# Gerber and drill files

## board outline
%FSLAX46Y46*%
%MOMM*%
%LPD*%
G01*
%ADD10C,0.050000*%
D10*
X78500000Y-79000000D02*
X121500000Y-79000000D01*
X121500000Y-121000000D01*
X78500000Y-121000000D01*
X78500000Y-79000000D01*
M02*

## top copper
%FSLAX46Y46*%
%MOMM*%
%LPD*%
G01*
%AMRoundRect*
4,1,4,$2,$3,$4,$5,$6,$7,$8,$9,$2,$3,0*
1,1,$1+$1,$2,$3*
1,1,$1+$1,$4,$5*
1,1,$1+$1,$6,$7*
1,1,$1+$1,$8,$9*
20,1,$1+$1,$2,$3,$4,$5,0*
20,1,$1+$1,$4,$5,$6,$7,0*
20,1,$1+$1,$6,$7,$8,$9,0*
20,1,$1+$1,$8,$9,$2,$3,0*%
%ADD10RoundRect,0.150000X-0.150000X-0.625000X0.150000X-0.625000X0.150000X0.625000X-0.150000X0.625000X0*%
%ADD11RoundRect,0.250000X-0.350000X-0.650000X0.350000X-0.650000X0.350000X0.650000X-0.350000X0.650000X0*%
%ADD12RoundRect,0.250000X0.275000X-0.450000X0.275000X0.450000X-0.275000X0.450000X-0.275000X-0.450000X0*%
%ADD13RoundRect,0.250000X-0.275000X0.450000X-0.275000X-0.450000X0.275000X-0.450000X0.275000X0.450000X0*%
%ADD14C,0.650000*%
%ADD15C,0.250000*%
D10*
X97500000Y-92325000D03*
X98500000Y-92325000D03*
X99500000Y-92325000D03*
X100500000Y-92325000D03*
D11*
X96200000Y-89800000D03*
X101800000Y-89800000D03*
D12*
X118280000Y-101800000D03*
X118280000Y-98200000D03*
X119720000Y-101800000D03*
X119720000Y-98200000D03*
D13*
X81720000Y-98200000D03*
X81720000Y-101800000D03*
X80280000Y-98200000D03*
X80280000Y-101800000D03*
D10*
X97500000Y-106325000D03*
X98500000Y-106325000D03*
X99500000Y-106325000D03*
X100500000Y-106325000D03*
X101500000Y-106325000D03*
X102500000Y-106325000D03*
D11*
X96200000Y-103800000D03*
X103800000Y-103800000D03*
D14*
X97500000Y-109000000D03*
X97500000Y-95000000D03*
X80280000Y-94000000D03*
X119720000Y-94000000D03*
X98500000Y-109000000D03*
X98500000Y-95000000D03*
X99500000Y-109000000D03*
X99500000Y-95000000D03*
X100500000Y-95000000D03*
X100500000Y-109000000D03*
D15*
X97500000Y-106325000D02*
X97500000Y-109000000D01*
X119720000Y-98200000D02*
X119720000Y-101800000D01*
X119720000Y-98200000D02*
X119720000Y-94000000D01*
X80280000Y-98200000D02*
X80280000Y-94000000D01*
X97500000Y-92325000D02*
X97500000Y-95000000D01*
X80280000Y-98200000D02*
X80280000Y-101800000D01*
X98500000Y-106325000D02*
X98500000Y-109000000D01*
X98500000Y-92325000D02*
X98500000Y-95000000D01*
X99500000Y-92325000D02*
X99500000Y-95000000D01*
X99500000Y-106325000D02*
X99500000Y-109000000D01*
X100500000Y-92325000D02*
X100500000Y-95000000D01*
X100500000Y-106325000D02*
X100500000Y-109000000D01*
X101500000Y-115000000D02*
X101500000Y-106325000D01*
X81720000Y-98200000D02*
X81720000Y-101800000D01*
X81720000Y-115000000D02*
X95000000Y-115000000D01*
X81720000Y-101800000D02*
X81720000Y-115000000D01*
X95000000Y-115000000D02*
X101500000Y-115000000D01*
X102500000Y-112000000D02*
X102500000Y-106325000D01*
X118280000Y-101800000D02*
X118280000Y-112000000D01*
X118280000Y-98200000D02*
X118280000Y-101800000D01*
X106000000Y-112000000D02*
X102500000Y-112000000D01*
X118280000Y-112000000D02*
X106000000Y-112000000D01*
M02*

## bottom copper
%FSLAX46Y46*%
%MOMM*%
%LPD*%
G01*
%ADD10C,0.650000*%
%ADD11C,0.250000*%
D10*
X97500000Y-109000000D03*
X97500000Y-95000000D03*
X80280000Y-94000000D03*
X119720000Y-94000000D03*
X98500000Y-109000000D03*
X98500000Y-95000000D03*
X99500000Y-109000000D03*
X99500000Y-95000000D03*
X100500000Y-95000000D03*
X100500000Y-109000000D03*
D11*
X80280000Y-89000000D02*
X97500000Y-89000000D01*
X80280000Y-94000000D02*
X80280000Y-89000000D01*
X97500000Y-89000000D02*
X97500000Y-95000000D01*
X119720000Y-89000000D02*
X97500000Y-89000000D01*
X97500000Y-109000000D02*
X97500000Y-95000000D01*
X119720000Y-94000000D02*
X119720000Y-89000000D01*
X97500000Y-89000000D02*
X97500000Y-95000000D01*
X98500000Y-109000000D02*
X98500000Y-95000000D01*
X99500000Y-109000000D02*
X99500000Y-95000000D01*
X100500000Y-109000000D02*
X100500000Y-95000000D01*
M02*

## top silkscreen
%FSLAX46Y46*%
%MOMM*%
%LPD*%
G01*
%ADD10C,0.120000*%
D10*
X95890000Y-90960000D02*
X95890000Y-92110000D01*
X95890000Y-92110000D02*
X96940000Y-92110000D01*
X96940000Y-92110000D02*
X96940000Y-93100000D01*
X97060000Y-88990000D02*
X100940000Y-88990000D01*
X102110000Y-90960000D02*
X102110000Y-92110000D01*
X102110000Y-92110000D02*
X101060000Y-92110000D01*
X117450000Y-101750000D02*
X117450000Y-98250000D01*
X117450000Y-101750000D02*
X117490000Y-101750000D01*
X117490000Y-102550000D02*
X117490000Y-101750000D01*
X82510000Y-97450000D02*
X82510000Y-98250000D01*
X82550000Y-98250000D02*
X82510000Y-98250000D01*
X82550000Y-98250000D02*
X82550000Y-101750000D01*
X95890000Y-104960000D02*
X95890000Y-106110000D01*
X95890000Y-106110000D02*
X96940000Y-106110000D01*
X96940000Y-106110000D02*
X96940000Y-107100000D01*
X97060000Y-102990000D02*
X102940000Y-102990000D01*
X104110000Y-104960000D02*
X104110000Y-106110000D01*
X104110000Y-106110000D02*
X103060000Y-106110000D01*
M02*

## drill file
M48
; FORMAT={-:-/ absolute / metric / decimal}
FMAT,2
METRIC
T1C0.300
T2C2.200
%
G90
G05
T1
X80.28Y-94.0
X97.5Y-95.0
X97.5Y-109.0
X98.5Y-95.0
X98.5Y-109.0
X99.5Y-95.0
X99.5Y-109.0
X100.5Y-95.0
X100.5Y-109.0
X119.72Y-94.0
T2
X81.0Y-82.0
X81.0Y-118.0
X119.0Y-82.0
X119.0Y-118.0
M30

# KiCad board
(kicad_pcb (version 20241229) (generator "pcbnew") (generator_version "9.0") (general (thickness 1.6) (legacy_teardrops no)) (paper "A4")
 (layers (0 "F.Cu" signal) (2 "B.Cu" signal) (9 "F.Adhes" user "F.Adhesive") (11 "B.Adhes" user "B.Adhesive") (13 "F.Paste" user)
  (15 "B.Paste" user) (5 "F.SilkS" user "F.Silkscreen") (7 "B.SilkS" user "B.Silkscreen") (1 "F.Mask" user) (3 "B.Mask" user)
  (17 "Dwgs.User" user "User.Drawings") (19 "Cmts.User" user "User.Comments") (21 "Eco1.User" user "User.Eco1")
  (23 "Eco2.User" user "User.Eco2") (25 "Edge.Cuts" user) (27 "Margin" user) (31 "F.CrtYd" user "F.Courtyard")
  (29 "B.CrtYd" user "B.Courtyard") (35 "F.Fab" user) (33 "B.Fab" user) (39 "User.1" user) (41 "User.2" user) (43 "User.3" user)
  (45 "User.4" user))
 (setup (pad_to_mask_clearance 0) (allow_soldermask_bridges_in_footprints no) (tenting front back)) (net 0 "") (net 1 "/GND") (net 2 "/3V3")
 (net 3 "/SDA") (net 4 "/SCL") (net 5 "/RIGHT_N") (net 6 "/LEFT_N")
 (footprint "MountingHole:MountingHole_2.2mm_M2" (layer "F.Cu") (at 119 82)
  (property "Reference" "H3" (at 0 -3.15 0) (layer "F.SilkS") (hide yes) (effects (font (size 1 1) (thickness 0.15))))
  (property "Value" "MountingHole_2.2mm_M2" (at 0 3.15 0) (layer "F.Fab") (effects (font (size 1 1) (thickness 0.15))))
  (pad "" np_thru_hole circle (at 0 0) (size 2.2 2.2) (drill 2.2) (layers "*.Cu" "*.Mask")))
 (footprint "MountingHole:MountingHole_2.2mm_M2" (layer "F.Cu") (at 81 82)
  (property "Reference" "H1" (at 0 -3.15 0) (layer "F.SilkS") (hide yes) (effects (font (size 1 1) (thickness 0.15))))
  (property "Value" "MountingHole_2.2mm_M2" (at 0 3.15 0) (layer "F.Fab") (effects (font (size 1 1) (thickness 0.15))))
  (pad "" np_thru_hole circle (at 0 0) (size 2.2 2.2) (drill 2.2) (layers "*.Cu" "*.Mask")))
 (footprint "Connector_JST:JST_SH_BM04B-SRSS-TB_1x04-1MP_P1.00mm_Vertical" (layer "F.Cu") (at 99 91)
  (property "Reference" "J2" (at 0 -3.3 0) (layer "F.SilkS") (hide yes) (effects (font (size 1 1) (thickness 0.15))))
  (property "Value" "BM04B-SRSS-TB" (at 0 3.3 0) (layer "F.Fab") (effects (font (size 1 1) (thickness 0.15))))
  (fp_line (start -3.11 -0.04) (end -3.11 1.11) (stroke (width 0.12) (type solid)) (layer "F.SilkS"))
  (fp_line (start -3.11 1.11) (end -2.06 1.11) (stroke (width 0.12) (type solid)) (layer "F.SilkS"))
  (fp_line (start -2.06 1.11) (end -2.06 2.1) (stroke (width 0.12) (type solid)) (layer "F.SilkS"))
  (fp_line (start -1.94 -2.01) (end 1.94 -2.01) (stroke (width 0.12) (type solid)) (layer "F.SilkS"))
  (fp_line (start 3.11 -0.04) (end 3.11 1.11) (stroke (width 0.12) (type solid)) (layer "F.SilkS"))
  (fp_line (start 3.11 1.11) (end 2.06 1.11) (stroke (width 0.12) (type solid)) (layer "F.SilkS"))
  (pad "1" smd roundrect (at -1.5 1.325) (size 0.6 1.55) (layers "F.Cu" "F.Mask" "F.Paste") (roundrect_rratio 0.25) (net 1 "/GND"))
  (pad "2" smd roundrect (at -0.5 1.325) (size 0.6 1.55) (layers "F.Cu" "F.Mask" "F.Paste") (roundrect_rratio 0.25) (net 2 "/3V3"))
  (pad "3" smd roundrect (at 0.5 1.325) (size 0.6 1.55) (layers "F.Cu" "F.Mask" "F.Paste") (roundrect_rratio 0.25) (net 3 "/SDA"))
  (pad "4" smd roundrect (at 1.5 1.325) (size 0.6 1.55) (layers "F.Cu" "F.Mask" "F.Paste") (roundrect_rratio 0.25) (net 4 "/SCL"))
  (pad "MP" smd roundrect (at -2.8 -1.2) (size 1.2 1.8) (layers "F.Cu" "F.Mask" "F.Paste") (roundrect_rratio 0.208333))
  (pad "MP" smd roundrect (at 2.8 -1.2) (size 1.2 1.8) (layers "F.Cu" "F.Mask" "F.Paste") (roundrect_rratio 0.208333)))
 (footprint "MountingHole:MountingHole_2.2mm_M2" (layer "F.Cu") (at 81 118)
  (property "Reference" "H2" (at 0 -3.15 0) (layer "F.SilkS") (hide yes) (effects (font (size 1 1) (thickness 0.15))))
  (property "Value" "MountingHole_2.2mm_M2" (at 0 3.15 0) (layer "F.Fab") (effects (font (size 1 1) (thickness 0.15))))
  (pad "" np_thru_hole circle (at 0 0) (size 2.2 2.2) (drill 2.2) (layers "*.Cu" "*.Mask")))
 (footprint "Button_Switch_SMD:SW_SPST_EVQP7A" (layer "F.Cu") (at 119 100 90)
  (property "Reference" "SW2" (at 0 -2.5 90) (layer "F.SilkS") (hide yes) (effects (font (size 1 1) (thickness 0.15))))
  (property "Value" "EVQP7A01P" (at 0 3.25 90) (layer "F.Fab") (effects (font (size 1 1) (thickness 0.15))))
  (fp_line (start -1.75 -1.55) (end 1.75 -1.55) (stroke (width 0.12) (type solid)) (layer "F.SilkS"))
  (fp_line (start -1.75 -1.55) (end -1.75 -1.51) (stroke (width 0.12) (type default)) (layer "F.SilkS"))
  (fp_line (start -2.55 -1.51) (end -1.75 -1.51) (stroke (width 0.12) (type default)) (layer "F.SilkS"))
  (pad "1" smd roundrect (at -1.8 -0.72 90) (size 1.4 1.05) (layers "F.Cu" "F.Mask" "F.Paste") (roundrect_rratio 0.2380952381)
   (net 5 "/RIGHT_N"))
  (pad "1" smd roundrect (at 1.8 -0.72 90) (size 1.4 1.05) (layers "F.Cu" "F.Mask" "F.Paste") (roundrect_rratio 0.2380952381)
   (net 5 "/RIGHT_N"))
  (pad "2" smd roundrect (at -1.8 0.72 90) (size 1.4 1.05) (layers "F.Cu" "F.Mask" "F.Paste") (roundrect_rratio 0.2380952381) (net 1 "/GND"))
  (pad "2" smd roundrect (at 1.8 0.72 90) (size 1.4 1.05) (layers "F.Cu" "F.Mask" "F.Paste") (roundrect_rratio 0.2380952381) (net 1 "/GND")))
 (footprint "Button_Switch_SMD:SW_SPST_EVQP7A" (layer "F.Cu") (at 81 100 -90)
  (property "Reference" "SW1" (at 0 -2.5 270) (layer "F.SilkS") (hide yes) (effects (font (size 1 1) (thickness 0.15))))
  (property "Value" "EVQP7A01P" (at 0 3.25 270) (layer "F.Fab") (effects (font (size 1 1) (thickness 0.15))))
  (fp_line (start -2.55 -1.51) (end -1.75 -1.51) (stroke (width 0.12) (type default)) (layer "F.SilkS"))
  (fp_line (start -1.75 -1.55) (end -1.75 -1.51) (stroke (width 0.12) (type default)) (layer "F.SilkS"))
  (fp_line (start -1.75 -1.55) (end 1.75 -1.55) (stroke (width 0.12) (type solid)) (layer "F.SilkS"))
  (pad "1" smd roundrect (at -1.8 -0.72 270) (size 1.4 1.05) (layers "F.Cu" "F.Mask" "F.Paste") (roundrect_rratio 0.2380952381)
   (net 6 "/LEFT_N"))
  (pad "1" smd roundrect (at 1.8 -0.72 270) (size 1.4 1.05) (layers "F.Cu" "F.Mask" "F.Paste") (roundrect_rratio 0.2380952381)
   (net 6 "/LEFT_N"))
  (pad "2" smd roundrect (at -1.8 0.72 270) (size 1.4 1.05) (layers "F.Cu" "F.Mask" "F.Paste") (roundrect_rratio 0.2380952381)
   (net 1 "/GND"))
  (pad "2" smd roundrect (at 1.8 0.72 270) (size 1.4 1.05) (layers "F.Cu" "F.Mask" "F.Paste") (roundrect_rratio 0.2380952381) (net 1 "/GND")))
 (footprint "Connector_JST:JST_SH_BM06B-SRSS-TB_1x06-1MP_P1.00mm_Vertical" (layer "F.Cu") (at 100 105)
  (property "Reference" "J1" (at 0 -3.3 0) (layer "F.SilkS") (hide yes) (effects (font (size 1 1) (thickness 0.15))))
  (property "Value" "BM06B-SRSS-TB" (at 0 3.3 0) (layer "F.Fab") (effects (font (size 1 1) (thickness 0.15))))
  (fp_line (start -4.11 -0.04) (end -4.11 1.11) (stroke (width 0.12) (type solid)) (layer "F.SilkS"))
  (fp_line (start -4.11 1.11) (end -3.06 1.11) (stroke (width 0.12) (type solid)) (layer "F.SilkS"))
  (fp_line (start -3.06 1.11) (end -3.06 2.1) (stroke (width 0.12) (type solid)) (layer "F.SilkS"))
  (fp_line (start -2.94 -2.01) (end 2.94 -2.01) (stroke (width 0.12) (type solid)) (layer "F.SilkS"))
  (fp_line (start 4.11 -0.04) (end 4.11 1.11) (stroke (width 0.12) (type solid)) (layer "F.SilkS"))
  (fp_line (start 4.11 1.11) (end 3.06 1.11) (stroke (width 0.12) (type solid)) (layer "F.SilkS"))
  (pad "1" smd roundrect (at -2.5 1.325) (size 0.6 1.55) (layers "F.Cu" "F.Mask" "F.Paste") (roundrect_rratio 0.25) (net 1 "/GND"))
  (pad "2" smd roundrect (at -1.5 1.325) (size 0.6 1.55) (layers "F.Cu" "F.Mask" "F.Paste") (roundrect_rratio 0.25) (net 2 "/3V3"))
  (pad "3" smd roundrect (at -0.5 1.325) (size 0.6 1.55) (layers "F.Cu" "F.Mask" "F.Paste") (roundrect_rratio 0.25) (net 3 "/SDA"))
  (pad "4" smd roundrect (at 0.5 1.325) (size 0.6 1.55) (layers "F.Cu" "F.Mask" "F.Paste") (roundrect_rratio 0.25) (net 4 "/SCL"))
  (pad "5" smd roundrect (at 1.5 1.325) (size 0.6 1.55) (layers "F.Cu" "F.Mask" "F.Paste") (roundrect_rratio 0.25) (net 6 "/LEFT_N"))
  (pad "6" smd roundrect (at 2.5 1.325) (size 0.6 1.55) (layers "F.Cu" "F.Mask" "F.Paste") (roundrect_rratio 0.25) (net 5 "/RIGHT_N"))
  (pad "MP" smd roundrect (at -3.8 -1.2) (size 1.2 1.8) (layers "F.Cu" "F.Mask" "F.Paste") (roundrect_rratio 0.208333))
  (pad "MP" smd roundrect (at 3.8 -1.2) (size 1.2 1.8) (layers "F.Cu" "F.Mask" "F.Paste") (roundrect_rratio 0.208333)))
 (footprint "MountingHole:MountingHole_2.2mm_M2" (layer "F.Cu") (at 119 118)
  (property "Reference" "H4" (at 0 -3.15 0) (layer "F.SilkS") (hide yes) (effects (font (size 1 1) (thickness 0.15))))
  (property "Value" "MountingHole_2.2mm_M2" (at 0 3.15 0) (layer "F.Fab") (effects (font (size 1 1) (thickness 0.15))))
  (pad "" np_thru_hole circle (at 0 0) (size 2.2 2.2) (drill 2.2) (layers "*.Cu" "*.Mask")))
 (gr_rect (start 78.5 79) (end 121.5 121) (stroke (width 0.05) (type default)) (fill no) (layer "Edge.Cuts"))
 (segment (start 97.5 106.325) (end 97.5 109) (width 0.25) (layer "F.Cu") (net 1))
 (segment (start 119.72 98.2) (end 119.72 101.8) (width 0.25) (layer "F.Cu") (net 1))
 (segment (start 119.72 98.2) (end 119.72 94) (width 0.25) (layer "F.Cu") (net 1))
 (segment (start 80.28 98.2) (end 80.28 94) (width 0.25) (layer "F.Cu") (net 1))
 (segment (start 97.5 92.325) (end 97.5 95) (width 0.25) (layer "F.Cu") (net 1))
 (segment (start 80.28 98.2) (end 80.28 101.8) (width 0.25) (layer "F.Cu") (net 1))
 (via (at 97.5 109) (size 0.65) (drill 0.3) (layers "F.Cu" "B.Cu") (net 1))
 (via (at 97.5 95) (size 0.65) (drill 0.3) (layers "F.Cu" "B.Cu") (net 1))
 (via (at 80.28 94) (size 0.65) (drill 0.3) (layers "F.Cu" "B.Cu") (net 1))
 (via (at 119.72 94) (size 0.65) (drill 0.3) (layers "F.Cu" "B.Cu") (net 1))
 (segment (start 80.28 89) (end 97.5 89) (width 0.25) (layer "B.Cu") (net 1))
 (segment (start 80.28 94) (end 80.28 89) (width 0.25) (layer "B.Cu") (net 1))
 (segment (start 97.5 89) (end 97.5 95) (width 0.25) (layer "B.Cu") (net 1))
 (segment (start 119.72 89) (end 97.5 89) (width 0.25) (layer "B.Cu") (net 1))
 (segment (start 97.5 109) (end 97.5 95) (width 0.25) (layer "B.Cu") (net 1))
 (segment (start 119.72 94) (end 119.72 89) (width 0.25) (layer "B.Cu") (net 1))
 (segment (start 97.5 89) (end 97.5 95) (width 0.25) (layer "B.Cu") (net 1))
 (segment (start 98.5 106.325) (end 98.5 109) (width 0.25) (layer "F.Cu") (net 2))
 (segment (start 98.5 92.325) (end 98.5 95) (width 0.25) (layer "F.Cu") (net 2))
 (via (at 98.5 109) (size 0.65) (drill 0.3) (layers "F.Cu" "B.Cu") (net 2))
 (via (at 98.5 95) (size 0.65) (drill 0.3) (layers "F.Cu" "B.Cu") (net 2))
 (segment (start 98.5 109) (end 98.5 95) (width 0.25) (layer "B.Cu") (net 2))
 (segment (start 99.5 92.325) (end 99.5 95) (width 0.25) (layer "F.Cu") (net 3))
 (segment (start 99.5 106.325) (end 99.5 109) (width 0.25) (layer "F.Cu") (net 3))
 (via (at 99.5 109) (size 0.65) (drill 0.3) (layers "F.Cu" "B.Cu") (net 3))
 (via (at 99.5 95) (size 0.65) (drill 0.3) (layers "F.Cu" "B.Cu") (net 3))
 (segment (start 99.5 109) (end 99.5 95) (width 0.25) (layer "B.Cu") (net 3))
 (segment (start 100.5 92.325) (end 100.5 95) (width 0.25) (layer "F.Cu") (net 4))
 (segment (start 100.5 106.325) (end 100.5 109) (width 0.25) (layer "F.Cu") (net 4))
 (via (at 100.5 95) (size 0.65) (drill 0.3) (layers "F.Cu" "B.Cu") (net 4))
 (via (at 100.5 109) (size 0.65) (drill 0.3) (layers "F.Cu" "B.Cu") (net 4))
 (segment (start 100.5 109) (end 100.5 95) (width 0.25) (layer "B.Cu") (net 4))
 (segment (start 101.5 115) (end 101.5 106.325) (width 0.25) (layer "F.Cu") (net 6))
 (segment (start 81.72 98.2) (end 81.72 101.8) (width 0.25) (layer "F.Cu") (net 6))
 (segment (start 81.72 115) (end 95 115) (width 0.25) (layer "F.Cu") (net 6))
 (segment (start 81.72 101.8) (end 81.72 115) (width 0.25) (layer "F.Cu") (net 6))
 (segment (start 95 115) (end 101.5 115) (width 0.25) (layer "F.Cu") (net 6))
 (segment (start 102.5 112) (end 102.5 106.325) (width 0.25) (layer "F.Cu") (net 5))
 (segment (start 118.28 101.8) (end 118.28 112) (width 0.25) (layer "F.Cu") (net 5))
 (segment (start 118.28 98.2) (end 118.28 101.8) (width 0.25) (layer "F.Cu") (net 5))
 (segment (start 106 112) (end 102.5 112) (width 0.25) (layer "F.Cu") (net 5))
 (segment (start 118.28 112) (end 106 112) (width 0.25) (layer "F.Cu") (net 5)))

